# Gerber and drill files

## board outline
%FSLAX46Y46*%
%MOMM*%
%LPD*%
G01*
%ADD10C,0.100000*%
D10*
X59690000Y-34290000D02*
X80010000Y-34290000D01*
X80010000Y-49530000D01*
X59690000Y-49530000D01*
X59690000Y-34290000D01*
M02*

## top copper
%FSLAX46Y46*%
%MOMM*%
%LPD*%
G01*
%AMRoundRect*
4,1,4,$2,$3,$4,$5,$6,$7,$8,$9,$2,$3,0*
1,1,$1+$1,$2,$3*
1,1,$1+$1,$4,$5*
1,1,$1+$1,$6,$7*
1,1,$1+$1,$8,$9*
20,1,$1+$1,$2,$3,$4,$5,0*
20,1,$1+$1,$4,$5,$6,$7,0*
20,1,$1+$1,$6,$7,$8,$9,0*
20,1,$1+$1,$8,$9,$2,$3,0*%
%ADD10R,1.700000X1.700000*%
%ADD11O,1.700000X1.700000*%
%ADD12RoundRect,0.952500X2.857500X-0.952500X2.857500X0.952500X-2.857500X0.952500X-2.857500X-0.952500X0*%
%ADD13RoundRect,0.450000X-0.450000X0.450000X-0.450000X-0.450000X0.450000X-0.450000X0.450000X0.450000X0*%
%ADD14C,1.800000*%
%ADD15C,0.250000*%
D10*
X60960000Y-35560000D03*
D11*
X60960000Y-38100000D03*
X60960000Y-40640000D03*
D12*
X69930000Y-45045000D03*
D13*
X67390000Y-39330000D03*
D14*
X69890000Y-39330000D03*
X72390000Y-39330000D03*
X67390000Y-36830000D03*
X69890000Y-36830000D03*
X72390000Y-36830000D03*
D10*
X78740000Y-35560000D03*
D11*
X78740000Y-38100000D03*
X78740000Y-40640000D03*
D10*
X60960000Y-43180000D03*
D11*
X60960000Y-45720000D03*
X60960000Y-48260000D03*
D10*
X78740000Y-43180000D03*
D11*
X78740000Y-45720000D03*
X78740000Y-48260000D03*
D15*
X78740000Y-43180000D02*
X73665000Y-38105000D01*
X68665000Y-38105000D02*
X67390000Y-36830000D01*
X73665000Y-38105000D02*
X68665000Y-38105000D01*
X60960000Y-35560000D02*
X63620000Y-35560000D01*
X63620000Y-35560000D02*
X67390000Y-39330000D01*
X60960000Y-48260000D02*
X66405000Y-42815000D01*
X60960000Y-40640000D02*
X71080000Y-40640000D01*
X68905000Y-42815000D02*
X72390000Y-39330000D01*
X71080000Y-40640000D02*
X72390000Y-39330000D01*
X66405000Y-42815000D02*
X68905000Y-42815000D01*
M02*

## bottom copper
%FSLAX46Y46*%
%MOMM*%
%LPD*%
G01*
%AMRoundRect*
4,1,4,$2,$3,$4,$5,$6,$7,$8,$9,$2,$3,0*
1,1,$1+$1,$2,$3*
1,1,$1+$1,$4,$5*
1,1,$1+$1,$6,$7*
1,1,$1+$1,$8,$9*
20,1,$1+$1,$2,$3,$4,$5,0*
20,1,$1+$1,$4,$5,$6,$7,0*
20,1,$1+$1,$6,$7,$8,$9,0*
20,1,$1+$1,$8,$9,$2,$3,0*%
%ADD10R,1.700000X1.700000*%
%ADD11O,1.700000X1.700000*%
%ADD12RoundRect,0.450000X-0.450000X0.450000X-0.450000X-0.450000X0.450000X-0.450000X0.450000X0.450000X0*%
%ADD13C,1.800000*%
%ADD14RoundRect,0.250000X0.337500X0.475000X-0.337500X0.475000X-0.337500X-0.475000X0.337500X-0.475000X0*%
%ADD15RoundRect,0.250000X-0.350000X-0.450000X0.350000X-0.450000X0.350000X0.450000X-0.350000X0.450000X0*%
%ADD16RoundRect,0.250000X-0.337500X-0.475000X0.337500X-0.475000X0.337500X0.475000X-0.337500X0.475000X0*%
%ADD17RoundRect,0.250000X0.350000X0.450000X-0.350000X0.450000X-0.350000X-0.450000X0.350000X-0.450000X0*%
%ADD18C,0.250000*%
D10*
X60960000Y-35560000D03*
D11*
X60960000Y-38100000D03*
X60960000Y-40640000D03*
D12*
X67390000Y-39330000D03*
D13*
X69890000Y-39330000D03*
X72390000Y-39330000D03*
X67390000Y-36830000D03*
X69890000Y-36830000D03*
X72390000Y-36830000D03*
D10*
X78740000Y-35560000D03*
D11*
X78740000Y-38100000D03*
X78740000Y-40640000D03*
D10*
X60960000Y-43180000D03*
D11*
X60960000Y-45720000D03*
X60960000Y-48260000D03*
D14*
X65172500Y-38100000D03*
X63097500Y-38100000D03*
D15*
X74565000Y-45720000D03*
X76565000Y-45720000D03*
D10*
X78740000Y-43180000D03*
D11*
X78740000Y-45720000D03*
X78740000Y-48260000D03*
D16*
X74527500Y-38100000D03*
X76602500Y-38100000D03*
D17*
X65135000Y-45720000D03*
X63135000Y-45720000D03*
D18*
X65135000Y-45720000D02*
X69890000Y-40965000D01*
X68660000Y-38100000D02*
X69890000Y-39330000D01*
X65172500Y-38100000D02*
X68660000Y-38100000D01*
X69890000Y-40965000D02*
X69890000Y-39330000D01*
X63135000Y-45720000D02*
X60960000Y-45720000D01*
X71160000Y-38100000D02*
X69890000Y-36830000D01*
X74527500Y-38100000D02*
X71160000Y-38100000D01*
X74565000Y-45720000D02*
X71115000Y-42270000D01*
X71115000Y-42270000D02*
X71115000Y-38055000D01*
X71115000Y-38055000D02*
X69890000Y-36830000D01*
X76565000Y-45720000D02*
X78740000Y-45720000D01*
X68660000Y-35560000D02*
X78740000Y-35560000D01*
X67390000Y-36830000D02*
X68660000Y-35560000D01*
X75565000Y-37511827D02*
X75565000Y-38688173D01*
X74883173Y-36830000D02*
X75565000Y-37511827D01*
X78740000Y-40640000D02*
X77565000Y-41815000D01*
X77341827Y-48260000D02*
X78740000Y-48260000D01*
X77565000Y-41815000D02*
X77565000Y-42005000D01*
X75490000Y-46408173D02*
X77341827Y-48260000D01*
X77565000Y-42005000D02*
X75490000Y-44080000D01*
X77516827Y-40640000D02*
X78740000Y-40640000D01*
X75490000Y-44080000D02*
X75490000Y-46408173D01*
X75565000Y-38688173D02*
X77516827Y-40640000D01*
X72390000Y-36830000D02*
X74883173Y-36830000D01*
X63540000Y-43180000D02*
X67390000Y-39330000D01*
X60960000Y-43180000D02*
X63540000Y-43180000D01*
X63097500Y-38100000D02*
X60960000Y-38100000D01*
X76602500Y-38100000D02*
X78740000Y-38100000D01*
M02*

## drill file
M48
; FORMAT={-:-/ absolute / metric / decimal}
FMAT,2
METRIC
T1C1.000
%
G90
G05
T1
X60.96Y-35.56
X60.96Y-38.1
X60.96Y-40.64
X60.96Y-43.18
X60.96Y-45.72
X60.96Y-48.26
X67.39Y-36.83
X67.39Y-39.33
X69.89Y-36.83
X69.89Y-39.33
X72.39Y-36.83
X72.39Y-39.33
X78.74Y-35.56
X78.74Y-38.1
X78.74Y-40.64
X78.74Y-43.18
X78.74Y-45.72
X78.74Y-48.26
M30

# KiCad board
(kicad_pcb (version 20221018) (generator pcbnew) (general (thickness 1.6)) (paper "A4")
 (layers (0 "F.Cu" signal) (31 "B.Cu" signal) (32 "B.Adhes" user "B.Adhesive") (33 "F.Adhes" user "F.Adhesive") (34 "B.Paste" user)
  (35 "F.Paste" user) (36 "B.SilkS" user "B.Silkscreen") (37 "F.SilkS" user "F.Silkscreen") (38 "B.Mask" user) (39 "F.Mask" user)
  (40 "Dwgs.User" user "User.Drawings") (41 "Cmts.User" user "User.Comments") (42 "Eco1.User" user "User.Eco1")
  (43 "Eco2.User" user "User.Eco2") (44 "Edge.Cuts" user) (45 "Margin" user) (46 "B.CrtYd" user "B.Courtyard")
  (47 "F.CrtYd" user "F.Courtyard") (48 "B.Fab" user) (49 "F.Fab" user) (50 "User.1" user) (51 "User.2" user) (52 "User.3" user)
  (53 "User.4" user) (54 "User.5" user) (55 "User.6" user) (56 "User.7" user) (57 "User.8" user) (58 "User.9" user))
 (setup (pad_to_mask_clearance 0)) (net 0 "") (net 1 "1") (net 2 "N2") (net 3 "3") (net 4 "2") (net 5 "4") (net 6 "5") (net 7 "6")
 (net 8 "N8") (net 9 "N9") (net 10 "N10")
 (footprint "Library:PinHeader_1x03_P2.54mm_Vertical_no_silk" (layer "F.Cu") (at 60.96 35.56)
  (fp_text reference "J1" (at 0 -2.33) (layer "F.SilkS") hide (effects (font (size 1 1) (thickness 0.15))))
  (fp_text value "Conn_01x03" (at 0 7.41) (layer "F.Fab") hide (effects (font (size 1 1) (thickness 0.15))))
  (pad "1" thru_hole rect (at 0 0) (size 1.7 1.7) (drill 1) (layers "*.Cu" "*.Mask") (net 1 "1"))
  (pad "2" thru_hole oval (at 0 2.54) (size 1.7 1.7) (drill 1) (layers "*.Cu" "*.Mask") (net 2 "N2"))
  (pad "3" thru_hole oval (at 0 5.08) (size 1.7 1.7) (drill 1) (layers "*.Cu" "*.Mask") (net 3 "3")))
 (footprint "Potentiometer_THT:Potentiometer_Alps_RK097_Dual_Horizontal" (layer "F.Cu") (at 67.39 39.33 90)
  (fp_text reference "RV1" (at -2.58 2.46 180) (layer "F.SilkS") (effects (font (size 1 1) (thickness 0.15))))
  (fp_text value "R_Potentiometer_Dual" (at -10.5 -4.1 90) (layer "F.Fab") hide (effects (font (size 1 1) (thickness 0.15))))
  (pad "" smd roundrect (at -5.715 2.54 90) (size 3.81 7.62) (layers "F.Cu" "F.Paste" "F.Mask") (roundrect_rratio 0.25))
  (pad "1" thru_hole roundrect (at 0 0 270) (size 1.8 1.8) (drill 1) (layers "*.Cu" "*.Mask") (roundrect_rratio 0.25) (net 1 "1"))
  (pad "2" thru_hole circle (at 0 2.5 270) (size 1.8 1.8) (drill 1) (layers "*.Cu" "*.Mask") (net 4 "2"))
  (pad "3" thru_hole circle (at 0 5 270) (size 1.8 1.8) (drill 1) (layers "*.Cu" "*.Mask") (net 3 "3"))
  (pad "4" thru_hole circle (at 2.5 0 270) (size 1.8 1.8) (drill 1) (layers "*.Cu" "*.Mask") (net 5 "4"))
  (pad "5" thru_hole circle (at 2.5 2.5 270) (size 1.8 1.8) (drill 1) (layers "*.Cu" "*.Mask") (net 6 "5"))
  (pad "6" thru_hole circle (at 2.5 5 270) (size 1.8 1.8) (drill 1) (layers "*.Cu" "*.Mask") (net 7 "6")))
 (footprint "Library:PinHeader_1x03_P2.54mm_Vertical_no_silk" (layer "F.Cu") (at 78.74 35.56)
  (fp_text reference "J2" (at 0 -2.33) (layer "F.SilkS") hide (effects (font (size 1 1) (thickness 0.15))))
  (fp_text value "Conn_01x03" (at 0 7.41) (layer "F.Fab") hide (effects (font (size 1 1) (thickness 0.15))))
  (pad "1" thru_hole rect (at 0 0) (size 1.7 1.7) (drill 1) (layers "*.Cu" "*.Mask") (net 5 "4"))
  (pad "2" thru_hole oval (at 0 2.54) (size 1.7 1.7) (drill 1) (layers "*.Cu" "*.Mask") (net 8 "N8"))
  (pad "3" thru_hole oval (at 0 5.08) (size 1.7 1.7) (drill 1) (layers "*.Cu" "*.Mask") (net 7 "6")))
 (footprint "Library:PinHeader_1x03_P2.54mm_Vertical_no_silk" (layer "B.Cu") (at 60.96 43.18 180)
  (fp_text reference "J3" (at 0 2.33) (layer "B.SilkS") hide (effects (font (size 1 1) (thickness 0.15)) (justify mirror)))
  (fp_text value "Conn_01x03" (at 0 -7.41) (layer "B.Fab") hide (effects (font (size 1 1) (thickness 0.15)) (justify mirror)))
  (pad "1" thru_hole rect (at 0 0 180) (size 1.7 1.7) (drill 1) (layers "*.Cu" "*.Mask") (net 1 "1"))
  (pad "2" thru_hole oval (at 0 -2.54 180) (size 1.7 1.7) (drill 1) (layers "*.Cu" "*.Mask") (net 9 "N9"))
  (pad "3" thru_hole oval (at 0 -5.08 180) (size 1.7 1.7) (drill 1) (layers "*.Cu" "*.Mask") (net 3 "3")))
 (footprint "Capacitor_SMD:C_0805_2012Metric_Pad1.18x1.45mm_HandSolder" (layer "B.Cu") (at 64.135 38.1 180)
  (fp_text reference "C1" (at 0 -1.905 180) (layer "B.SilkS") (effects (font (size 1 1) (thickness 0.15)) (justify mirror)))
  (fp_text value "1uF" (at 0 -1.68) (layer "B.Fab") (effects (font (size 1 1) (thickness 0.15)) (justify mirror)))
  (pad "1" smd roundrect (at -1.0375 0 180) (size 1.175 1.45) (layers "B.Cu" "B.Paste" "B.Mask") (roundrect_rratio 0.212766) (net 4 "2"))
  (pad "2" smd roundrect (at 1.0375 0 180) (size 1.175 1.45) (layers "B.Cu" "B.Paste" "B.Mask") (roundrect_rratio 0.212766) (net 2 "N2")))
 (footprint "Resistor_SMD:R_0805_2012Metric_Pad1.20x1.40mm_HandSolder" (layer "B.Cu") (at 75.565 45.72)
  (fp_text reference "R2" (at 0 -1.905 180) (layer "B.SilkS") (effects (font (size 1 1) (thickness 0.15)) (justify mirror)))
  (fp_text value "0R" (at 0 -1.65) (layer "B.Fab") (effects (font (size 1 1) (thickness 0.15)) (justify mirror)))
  (pad "1" smd roundrect (at -1 0) (size 1.2 1.4) (layers "B.Cu" "B.Paste" "B.Mask") (roundrect_rratio 0.208333) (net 6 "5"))
  (pad "2" smd roundrect (at 1 0) (size 1.2 1.4) (layers "B.Cu" "B.Paste" "B.Mask") (roundrect_rratio 0.208333) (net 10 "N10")))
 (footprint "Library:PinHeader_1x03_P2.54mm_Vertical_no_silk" (layer "B.Cu") (at 78.74 43.18 180)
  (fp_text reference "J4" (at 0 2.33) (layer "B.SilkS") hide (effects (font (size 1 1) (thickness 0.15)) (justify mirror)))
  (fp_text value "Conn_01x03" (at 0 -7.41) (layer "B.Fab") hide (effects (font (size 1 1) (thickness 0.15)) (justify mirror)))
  (pad "1" thru_hole rect (at 0 0 180) (size 1.7 1.7) (drill 1) (layers "*.Cu" "*.Mask") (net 5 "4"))
  (pad "2" thru_hole oval (at 0 -2.54 180) (size 1.7 1.7) (drill 1) (layers "*.Cu" "*.Mask") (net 10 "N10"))
  (pad "3" thru_hole oval (at 0 -5.08 180) (size 1.7 1.7) (drill 1) (layers "*.Cu" "*.Mask") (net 7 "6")))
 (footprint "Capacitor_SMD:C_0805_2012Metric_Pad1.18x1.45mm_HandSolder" (layer "B.Cu") (at 75.565 38.1)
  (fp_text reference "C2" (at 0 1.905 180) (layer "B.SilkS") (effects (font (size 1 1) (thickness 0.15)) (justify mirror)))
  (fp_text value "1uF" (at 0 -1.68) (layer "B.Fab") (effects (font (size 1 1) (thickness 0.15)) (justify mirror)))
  (pad "1" smd roundrect (at -1.0375 0) (size 1.175 1.45) (layers "B.Cu" "B.Paste" "B.Mask") (roundrect_rratio 0.212766) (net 6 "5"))
  (pad "2" smd roundrect (at 1.0375 0) (size 1.175 1.45) (layers "B.Cu" "B.Paste" "B.Mask") (roundrect_rratio 0.212766) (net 8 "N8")))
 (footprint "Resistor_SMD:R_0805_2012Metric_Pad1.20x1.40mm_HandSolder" (layer "B.Cu") (at 64.135 45.72 180)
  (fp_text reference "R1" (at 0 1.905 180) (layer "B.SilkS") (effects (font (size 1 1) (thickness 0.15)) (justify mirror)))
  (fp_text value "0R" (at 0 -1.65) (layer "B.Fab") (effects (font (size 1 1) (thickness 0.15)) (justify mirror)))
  (pad "1" smd roundrect (at -1 0 180) (size 1.2 1.4) (layers "B.Cu" "B.Paste" "B.Mask") (roundrect_rratio 0.208333) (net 4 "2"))
  (pad "2" smd roundrect (at 1 0 180) (size 1.2 1.4) (layers "B.Cu" "B.Paste" "B.Mask") (roundrect_rratio 0.208333) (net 9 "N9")))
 (gr_rect (start 59.69 34.29) (end 80.01 49.53) (stroke (width 0.1) (type default)) (fill none) (layer "Edge.Cuts"))
 (segment (start 65.135 45.72) (end 69.89 40.965) (width 0.25) (layer "B.Cu") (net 4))
 (segment (start 68.66 38.1) (end 69.89 39.33) (width 0.25) (layer "B.Cu") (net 4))
 (segment (start 65.1725 38.1) (end 68.66 38.1) (width 0.25) (layer "B.Cu") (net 4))
 (segment (start 69.89 40.965) (end 69.89 39.33) (width 0.25) (layer "B.Cu") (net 4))
 (segment (start 63.135 45.72) (end 60.96 45.72) (width 0.25) (layer "B.Cu") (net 9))
 (segment (start 71.16 38.1) (end 69.89 36.83) (width 0.25) (layer "B.Cu") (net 6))
 (segment (start 74.5275 38.1) (end 71.16 38.1) (width 0.25) (layer "B.Cu") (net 6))
 (segment (start 74.565 45.72) (end 71.115 42.27) (width 0.25) (layer "B.Cu") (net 6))
 (segment (start 71.115 42.27) (end 71.115 38.055) (width 0.25) (layer "B.Cu") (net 6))
 (segment (start 71.115 38.055) (end 69.89 36.83) (width 0.25) (layer "B.Cu") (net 6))
 (segment (start 76.565 45.72) (end 78.74 45.72) (width 0.25) (layer "B.Cu") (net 10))
 (segment (start 78.74 43.18) (end 73.665 38.105) (width 0.25) (layer "F.Cu") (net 5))
 (segment (start 68.665 38.105) (end 67.39 36.83) (width 0.25) (layer "F.Cu") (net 5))
 (segment (start 73.665 38.105) (end 68.665 38.105) (width 0.25) (layer "F.Cu") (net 5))
 (segment (start 68.66 35.56) (end 78.74 35.56) (width 0.25) (layer "B.Cu") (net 5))
 (segment (start 67.39 36.83) (end 68.66 35.56) (width 0.25) (layer "B.Cu") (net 5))
 (segment (start 75.565 37.511827) (end 75.565 38.688173) (width 0.25) (layer "B.Cu") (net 7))
 (segment (start 74.883173 36.83) (end 75.565 37.511827) (width 0.25) (layer "B.Cu") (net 7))
 (segment (start 78.74 40.64) (end 77.565 41.815) (width 0.25) (layer "B.Cu") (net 7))
 (segment (start 77.341827 48.26) (end 78.74 48.26) (width 0.25) (layer "B.Cu") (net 7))
 (segment (start 77.565 41.815) (end 77.565 42.005) (width 0.25) (layer "B.Cu") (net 7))
 (segment (start 75.49 46.408173) (end 77.341827 48.26) (width 0.25) (layer "B.Cu") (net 7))
 (segment (start 77.565 42.005) (end 75.49 44.08) (width 0.25) (layer "B.Cu") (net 7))
 (segment (start 77.516827 40.64) (end 78.74 40.64) (width 0.25) (layer "B.Cu") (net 7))
 (segment (start 75.49 44.08) (end 75.49 46.408173) (width 0.25) (layer "B.Cu") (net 7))
 (segment (start 75.565 38.688173) (end 77.516827 40.64) (width 0.25) (layer "B.Cu") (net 7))
 (segment (start 72.39 36.83) (end 74.883173 36.83) (width 0.25) (layer "B.Cu") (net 7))
 (segment (start 60.96 35.56) (end 63.62 35.56) (width 0.25) (layer "F.Cu") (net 1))
 (segment (start 63.62 35.56) (end 67.39 39.33) (width 0.25) (layer "F.Cu") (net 1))
 (segment (start 63.54 43.18) (end 67.39 39.33) (width 0.25) (layer "B.Cu") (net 1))
 (segment (start 60.96 43.18) (end 63.54 43.18) (width 0.25) (layer "B.Cu") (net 1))
 (segment (start 60.96 48.26) (end 66.405 42.815) (width 0.25) (layer "F.Cu") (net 3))
 (segment (start 60.96 40.64) (end 71.08 40.64) (width 0.25) (layer "F.Cu") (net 3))
 (segment (start 68.905 42.815) (end 72.39 39.33) (width 0.25) (layer "F.Cu") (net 3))
 (segment (start 71.08 40.64) (end 72.39 39.33) (width 0.25) (layer "F.Cu") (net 3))
 (segment (start 66.405 42.815) (end 68.905 42.815) (width 0.25) (layer "F.Cu") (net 3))
 (segment (start 63.0975 38.1) (end 60.96 38.1) (width 0.25) (layer "B.Cu") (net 2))
 (segment (start 76.6025 38.1) (end 78.74 38.1) (width 0.25) (layer "B.Cu") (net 8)))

